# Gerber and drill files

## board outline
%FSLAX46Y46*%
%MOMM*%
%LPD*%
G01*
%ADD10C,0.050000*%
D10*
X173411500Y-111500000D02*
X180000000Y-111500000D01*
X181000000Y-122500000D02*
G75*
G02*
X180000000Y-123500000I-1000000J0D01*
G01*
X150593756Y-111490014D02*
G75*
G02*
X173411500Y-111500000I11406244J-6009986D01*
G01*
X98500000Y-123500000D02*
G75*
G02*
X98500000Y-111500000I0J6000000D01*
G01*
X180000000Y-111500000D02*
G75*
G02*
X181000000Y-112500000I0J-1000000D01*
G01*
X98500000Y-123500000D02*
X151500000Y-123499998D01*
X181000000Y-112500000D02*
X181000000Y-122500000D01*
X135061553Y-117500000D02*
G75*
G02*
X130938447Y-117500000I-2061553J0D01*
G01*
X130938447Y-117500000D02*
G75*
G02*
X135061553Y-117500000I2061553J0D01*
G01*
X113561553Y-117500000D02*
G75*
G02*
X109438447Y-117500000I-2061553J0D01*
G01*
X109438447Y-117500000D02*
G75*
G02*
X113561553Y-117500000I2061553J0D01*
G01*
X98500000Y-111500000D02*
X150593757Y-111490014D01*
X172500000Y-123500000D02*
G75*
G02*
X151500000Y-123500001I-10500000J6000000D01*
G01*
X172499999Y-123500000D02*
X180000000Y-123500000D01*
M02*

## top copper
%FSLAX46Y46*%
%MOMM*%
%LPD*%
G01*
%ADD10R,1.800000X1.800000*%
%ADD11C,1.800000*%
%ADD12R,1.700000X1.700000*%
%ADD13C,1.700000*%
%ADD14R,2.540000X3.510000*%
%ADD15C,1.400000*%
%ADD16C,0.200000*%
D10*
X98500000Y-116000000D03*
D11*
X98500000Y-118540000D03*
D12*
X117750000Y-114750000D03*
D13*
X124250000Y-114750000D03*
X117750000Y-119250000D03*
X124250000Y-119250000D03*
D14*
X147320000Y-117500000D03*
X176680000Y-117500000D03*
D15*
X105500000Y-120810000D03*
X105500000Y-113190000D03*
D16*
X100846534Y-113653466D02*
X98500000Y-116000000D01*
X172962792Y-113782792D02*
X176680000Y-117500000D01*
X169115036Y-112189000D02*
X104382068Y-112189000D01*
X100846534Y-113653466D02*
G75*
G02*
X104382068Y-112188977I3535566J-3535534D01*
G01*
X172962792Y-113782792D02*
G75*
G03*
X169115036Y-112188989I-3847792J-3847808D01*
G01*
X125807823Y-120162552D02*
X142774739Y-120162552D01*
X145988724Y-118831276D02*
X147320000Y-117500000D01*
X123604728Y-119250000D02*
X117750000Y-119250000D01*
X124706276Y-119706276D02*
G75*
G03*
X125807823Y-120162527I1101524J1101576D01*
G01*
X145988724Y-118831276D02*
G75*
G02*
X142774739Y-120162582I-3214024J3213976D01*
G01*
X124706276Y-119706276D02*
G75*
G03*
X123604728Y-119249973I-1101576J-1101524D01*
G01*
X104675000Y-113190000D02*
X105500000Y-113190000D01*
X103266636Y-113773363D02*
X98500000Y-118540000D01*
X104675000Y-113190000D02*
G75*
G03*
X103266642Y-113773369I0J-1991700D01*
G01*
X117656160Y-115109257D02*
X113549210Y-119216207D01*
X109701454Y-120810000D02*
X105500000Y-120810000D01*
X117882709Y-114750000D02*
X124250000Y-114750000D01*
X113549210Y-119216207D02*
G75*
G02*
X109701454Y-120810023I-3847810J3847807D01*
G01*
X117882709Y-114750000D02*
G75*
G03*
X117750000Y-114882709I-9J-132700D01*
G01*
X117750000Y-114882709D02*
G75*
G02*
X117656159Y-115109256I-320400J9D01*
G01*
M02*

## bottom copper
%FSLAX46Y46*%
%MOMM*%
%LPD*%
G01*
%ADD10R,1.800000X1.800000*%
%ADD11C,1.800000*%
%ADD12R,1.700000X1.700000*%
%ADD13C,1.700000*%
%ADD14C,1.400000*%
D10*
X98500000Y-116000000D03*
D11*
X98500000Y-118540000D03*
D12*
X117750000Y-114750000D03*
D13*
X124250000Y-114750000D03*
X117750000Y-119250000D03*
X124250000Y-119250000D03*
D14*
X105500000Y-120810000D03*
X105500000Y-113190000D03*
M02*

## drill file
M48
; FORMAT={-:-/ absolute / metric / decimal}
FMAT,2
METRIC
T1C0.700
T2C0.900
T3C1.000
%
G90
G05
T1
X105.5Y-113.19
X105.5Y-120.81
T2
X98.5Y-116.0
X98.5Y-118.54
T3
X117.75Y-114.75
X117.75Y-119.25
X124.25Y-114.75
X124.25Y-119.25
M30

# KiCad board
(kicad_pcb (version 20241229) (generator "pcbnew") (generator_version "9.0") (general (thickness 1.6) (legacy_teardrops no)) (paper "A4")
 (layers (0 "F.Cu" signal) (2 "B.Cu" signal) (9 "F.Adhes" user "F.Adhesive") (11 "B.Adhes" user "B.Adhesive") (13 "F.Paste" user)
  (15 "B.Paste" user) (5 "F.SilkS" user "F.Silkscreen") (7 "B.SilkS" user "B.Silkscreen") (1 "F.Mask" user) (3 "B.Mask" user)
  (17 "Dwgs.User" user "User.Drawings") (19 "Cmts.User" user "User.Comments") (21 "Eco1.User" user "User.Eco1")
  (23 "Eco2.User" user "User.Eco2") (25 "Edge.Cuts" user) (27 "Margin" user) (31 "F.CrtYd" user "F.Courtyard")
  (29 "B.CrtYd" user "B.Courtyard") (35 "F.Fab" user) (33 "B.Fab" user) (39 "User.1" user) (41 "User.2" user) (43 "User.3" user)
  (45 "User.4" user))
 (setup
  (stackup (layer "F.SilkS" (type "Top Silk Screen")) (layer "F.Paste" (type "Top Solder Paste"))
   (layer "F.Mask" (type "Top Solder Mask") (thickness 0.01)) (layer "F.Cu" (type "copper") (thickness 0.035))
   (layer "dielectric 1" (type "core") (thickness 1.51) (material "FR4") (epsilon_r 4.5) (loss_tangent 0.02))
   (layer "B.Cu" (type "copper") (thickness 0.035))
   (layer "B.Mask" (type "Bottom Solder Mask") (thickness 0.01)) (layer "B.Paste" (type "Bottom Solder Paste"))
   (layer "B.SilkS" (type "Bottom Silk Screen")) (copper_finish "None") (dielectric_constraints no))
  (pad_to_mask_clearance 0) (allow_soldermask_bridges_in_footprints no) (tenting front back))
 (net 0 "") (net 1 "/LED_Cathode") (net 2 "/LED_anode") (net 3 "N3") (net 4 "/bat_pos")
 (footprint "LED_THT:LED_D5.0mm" (layer "F.Cu") (at 98.5 116 -90)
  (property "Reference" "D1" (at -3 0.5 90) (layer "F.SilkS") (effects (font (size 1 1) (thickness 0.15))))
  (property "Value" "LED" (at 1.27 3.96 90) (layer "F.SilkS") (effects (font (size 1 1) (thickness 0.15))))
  (pad "1" thru_hole rect (at 0 0 270) (size 1.8 1.8) (drill 0.9) (layers "*.Cu" "*.Mask") (remove_unused_layers no) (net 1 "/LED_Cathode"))
  (pad "2" thru_hole circle (at 2.54 0 270) (size 1.8 1.8) (drill 0.9) (layers "*.Cu" "*.Mask") (remove_unused_layers no)
   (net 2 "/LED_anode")))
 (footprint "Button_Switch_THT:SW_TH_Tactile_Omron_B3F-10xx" (layer "F.Cu") (at 117.75 114.75)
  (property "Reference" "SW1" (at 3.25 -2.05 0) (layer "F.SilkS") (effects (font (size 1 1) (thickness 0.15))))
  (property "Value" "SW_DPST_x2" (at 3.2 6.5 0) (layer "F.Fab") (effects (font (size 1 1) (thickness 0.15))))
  (pad "1" thru_hole rect (at 0 0) (size 1.7 1.7) (drill 1) (layers "*.Cu" "*.Mask") (remove_unused_layers no) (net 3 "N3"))
  (pad "1" thru_hole circle (at 6.5 0) (size 1.7 1.7) (drill 1) (layers "*.Cu" "*.Mask") (remove_unused_layers no) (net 3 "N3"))
  (pad "2" thru_hole circle (at 0 4.5) (size 1.7 1.7) (drill 1) (layers "*.Cu" "*.Mask") (remove_unused_layers no) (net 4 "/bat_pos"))
  (pad "2" thru_hole circle (at 6.5 4.5) (size 1.7 1.7) (drill 1) (layers "*.Cu" "*.Mask") (remove_unused_layers no) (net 4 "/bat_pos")))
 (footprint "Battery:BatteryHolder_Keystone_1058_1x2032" (layer "F.Cu") (at 162 117.5)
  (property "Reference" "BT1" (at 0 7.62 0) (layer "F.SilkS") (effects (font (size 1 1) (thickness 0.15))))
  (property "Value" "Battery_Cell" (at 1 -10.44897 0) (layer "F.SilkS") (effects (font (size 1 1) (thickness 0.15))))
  (pad "1" smd rect (at -14.68 0) (size 2.54 3.51) (layers "F.Cu" "F.Mask" "F.Paste") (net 4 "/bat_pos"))
  (pad "2" smd rect (at 14.68 0) (size 2.54 3.51) (layers "F.Cu" "F.Mask" "F.Paste") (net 1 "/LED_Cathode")))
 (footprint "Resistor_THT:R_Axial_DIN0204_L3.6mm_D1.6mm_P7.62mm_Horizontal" (layer "F.Cu") (at 105.5 120.81 90)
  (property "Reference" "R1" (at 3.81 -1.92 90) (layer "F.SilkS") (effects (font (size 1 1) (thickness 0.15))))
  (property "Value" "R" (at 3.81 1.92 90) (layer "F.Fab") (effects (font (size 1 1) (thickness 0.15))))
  (pad "1" thru_hole circle (at 0 0 90) (size 1.4 1.4) (drill 0.7) (layers "*.Cu" "*.Mask") (remove_unused_layers no) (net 3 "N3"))
  (pad "2" thru_hole circle (at 7.62 0 90) (size 1.4 1.4) (drill 0.7) (layers "*.Cu" "*.Mask") (remove_unused_layers no)
   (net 2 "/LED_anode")))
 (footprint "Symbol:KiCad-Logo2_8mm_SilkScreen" (layer "B.Cu") (at 163 117 180)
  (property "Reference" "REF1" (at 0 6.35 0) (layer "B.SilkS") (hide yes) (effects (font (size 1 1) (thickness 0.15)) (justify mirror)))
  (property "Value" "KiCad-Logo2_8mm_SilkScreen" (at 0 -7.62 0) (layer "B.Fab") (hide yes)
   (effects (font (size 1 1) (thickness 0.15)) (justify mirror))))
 (gr_line (start 173.4115 111.5) (end 180 111.5) (stroke (width 0.05) (type default)) (layer "Edge.Cuts"))
 (gr_arc (start 181 122.5) (mid 180.707107 123.207107) (end 180 123.5) (stroke (width 0.05) (type default)) (layer "Edge.Cuts"))
 (gr_arc (start 150.593756 111.490014) (mid 162.005642 104.607277) (end 173.4115 111.5) (stroke (width 0.05) (type default))
  (layer "Edge.Cuts"))
 (gr_arc (start 98.5 123.5) (mid 92.5 117.5) (end 98.5 111.5) (stroke (width 0.05) (type default)) (layer "Edge.Cuts"))
 (gr_arc (start 180 111.5) (mid 180.707107 111.792893) (end 181 112.5) (stroke (width 0.05) (type default)) (layer "Edge.Cuts"))
 (gr_line (start 98.5 123.5) (end 151.5 123.499998) (stroke (width 0.05) (type default)) (layer "Edge.Cuts"))
 (gr_line (start 181 112.5) (end 181 122.5) (stroke (width 0.05) (type default)) (layer "Edge.Cuts"))
 (gr_circle (center 133 117.5) (end 135 118) (stroke (width 0.05) (type default)) (fill no) (layer "Edge.Cuts"))
 (gr_circle (center 111.5 117.5) (end 113.5 118) (stroke (width 0.05) (type default)) (fill no) (layer "Edge.Cuts"))
 (gr_line (start 98.5 111.5) (end 150.593757 111.490014) (stroke (width 0.05) (type default)) (layer "Edge.Cuts"))
 (gr_arc (start 172.5 123.5) (mid 162 129.593387) (end 151.5 123.500001) (stroke (width 0.05) (type default)) (layer "Edge.Cuts"))
 (gr_line (start 172.499999 123.5) (end 180 123.5) (stroke (width 0.05) (type default)) (layer "Edge.Cuts"))
 (segment (start 100.846534 113.653466) (end 98.5 116) (width 0.2) (layer "F.Cu") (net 1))
 (segment (start 172.962792 113.782792) (end 176.68 117.5) (width 0.2) (layer "F.Cu") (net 1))
 (segment (start 169.115036 112.189) (end 104.382068 112.189) (width 0.2) (layer "F.Cu") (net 1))
 (arc (start 100.846534 113.653466) (mid 102.468651 112.569602) (end 104.382068 112.189) (width 0.2) (layer "F.Cu") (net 1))
 (arc (start 172.962792 113.782792) (mid 171.197426 112.603213) (end 169.115036 112.189) (width 0.2) (layer "F.Cu") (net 1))
 (segment (start 125.807823 120.162552) (end 142.774739 120.162552) (width 0.2) (layer "F.Cu") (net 4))
 (segment (start 145.988724 118.831276) (end 147.32 117.5) (width 0.2) (layer "F.Cu") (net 4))
 (segment (start 123.604728 119.25) (end 117.75 119.25) (width 0.2) (layer "F.Cu") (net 4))
 (arc (start 124.706276 119.706276) (mid 125.21167 120.043969) (end 125.807823 120.162552) (width 0.2) (layer "F.Cu") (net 4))
 (arc (start 145.988724 118.831276) (mid 144.514135 119.816564) (end 142.774739 120.162552) (width 0.2) (layer "F.Cu") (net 4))
 (arc (start 124.706276 119.706276) (mid 124.200881 119.368582) (end 123.604728 119.25) (width 0.2) (layer "F.Cu") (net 4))
 (segment (start 104.675 113.19) (end 105.5 113.19) (width 0.2) (layer "F.Cu") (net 2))
 (segment (start 103.266636 113.773363) (end 98.5 118.54) (width 0.2) (layer "F.Cu") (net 2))
 (arc (start 104.675 113.19) (mid 103.912799 113.341611) (end 103.266636 113.773363) (width 0.2) (layer "F.Cu") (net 2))
 (segment (start 117.65616 115.109257) (end 113.54921 119.216207) (width 0.2) (layer "F.Cu") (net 3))
 (segment (start 109.701454 120.81) (end 105.5 120.81) (width 0.2) (layer "F.Cu") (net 3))
 (segment (start 117.882709 114.75) (end 124.25 114.75) (width 0.2) (layer "F.Cu") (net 3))
 (arc (start 113.54921 119.216207) (mid 111.783844 120.395786) (end 109.701454 120.81) (width 0.2) (layer "F.Cu") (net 3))
 (arc (start 117.882709 114.75) (mid 117.788869 114.788869) (end 117.75 114.882709) (width 0.2) (layer "F.Cu") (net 3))
 (arc (start 117.75 114.882709) (mid 117.725611 115.005316) (end 117.65616 115.109257) (width 0.2) (layer "F.Cu") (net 3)))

